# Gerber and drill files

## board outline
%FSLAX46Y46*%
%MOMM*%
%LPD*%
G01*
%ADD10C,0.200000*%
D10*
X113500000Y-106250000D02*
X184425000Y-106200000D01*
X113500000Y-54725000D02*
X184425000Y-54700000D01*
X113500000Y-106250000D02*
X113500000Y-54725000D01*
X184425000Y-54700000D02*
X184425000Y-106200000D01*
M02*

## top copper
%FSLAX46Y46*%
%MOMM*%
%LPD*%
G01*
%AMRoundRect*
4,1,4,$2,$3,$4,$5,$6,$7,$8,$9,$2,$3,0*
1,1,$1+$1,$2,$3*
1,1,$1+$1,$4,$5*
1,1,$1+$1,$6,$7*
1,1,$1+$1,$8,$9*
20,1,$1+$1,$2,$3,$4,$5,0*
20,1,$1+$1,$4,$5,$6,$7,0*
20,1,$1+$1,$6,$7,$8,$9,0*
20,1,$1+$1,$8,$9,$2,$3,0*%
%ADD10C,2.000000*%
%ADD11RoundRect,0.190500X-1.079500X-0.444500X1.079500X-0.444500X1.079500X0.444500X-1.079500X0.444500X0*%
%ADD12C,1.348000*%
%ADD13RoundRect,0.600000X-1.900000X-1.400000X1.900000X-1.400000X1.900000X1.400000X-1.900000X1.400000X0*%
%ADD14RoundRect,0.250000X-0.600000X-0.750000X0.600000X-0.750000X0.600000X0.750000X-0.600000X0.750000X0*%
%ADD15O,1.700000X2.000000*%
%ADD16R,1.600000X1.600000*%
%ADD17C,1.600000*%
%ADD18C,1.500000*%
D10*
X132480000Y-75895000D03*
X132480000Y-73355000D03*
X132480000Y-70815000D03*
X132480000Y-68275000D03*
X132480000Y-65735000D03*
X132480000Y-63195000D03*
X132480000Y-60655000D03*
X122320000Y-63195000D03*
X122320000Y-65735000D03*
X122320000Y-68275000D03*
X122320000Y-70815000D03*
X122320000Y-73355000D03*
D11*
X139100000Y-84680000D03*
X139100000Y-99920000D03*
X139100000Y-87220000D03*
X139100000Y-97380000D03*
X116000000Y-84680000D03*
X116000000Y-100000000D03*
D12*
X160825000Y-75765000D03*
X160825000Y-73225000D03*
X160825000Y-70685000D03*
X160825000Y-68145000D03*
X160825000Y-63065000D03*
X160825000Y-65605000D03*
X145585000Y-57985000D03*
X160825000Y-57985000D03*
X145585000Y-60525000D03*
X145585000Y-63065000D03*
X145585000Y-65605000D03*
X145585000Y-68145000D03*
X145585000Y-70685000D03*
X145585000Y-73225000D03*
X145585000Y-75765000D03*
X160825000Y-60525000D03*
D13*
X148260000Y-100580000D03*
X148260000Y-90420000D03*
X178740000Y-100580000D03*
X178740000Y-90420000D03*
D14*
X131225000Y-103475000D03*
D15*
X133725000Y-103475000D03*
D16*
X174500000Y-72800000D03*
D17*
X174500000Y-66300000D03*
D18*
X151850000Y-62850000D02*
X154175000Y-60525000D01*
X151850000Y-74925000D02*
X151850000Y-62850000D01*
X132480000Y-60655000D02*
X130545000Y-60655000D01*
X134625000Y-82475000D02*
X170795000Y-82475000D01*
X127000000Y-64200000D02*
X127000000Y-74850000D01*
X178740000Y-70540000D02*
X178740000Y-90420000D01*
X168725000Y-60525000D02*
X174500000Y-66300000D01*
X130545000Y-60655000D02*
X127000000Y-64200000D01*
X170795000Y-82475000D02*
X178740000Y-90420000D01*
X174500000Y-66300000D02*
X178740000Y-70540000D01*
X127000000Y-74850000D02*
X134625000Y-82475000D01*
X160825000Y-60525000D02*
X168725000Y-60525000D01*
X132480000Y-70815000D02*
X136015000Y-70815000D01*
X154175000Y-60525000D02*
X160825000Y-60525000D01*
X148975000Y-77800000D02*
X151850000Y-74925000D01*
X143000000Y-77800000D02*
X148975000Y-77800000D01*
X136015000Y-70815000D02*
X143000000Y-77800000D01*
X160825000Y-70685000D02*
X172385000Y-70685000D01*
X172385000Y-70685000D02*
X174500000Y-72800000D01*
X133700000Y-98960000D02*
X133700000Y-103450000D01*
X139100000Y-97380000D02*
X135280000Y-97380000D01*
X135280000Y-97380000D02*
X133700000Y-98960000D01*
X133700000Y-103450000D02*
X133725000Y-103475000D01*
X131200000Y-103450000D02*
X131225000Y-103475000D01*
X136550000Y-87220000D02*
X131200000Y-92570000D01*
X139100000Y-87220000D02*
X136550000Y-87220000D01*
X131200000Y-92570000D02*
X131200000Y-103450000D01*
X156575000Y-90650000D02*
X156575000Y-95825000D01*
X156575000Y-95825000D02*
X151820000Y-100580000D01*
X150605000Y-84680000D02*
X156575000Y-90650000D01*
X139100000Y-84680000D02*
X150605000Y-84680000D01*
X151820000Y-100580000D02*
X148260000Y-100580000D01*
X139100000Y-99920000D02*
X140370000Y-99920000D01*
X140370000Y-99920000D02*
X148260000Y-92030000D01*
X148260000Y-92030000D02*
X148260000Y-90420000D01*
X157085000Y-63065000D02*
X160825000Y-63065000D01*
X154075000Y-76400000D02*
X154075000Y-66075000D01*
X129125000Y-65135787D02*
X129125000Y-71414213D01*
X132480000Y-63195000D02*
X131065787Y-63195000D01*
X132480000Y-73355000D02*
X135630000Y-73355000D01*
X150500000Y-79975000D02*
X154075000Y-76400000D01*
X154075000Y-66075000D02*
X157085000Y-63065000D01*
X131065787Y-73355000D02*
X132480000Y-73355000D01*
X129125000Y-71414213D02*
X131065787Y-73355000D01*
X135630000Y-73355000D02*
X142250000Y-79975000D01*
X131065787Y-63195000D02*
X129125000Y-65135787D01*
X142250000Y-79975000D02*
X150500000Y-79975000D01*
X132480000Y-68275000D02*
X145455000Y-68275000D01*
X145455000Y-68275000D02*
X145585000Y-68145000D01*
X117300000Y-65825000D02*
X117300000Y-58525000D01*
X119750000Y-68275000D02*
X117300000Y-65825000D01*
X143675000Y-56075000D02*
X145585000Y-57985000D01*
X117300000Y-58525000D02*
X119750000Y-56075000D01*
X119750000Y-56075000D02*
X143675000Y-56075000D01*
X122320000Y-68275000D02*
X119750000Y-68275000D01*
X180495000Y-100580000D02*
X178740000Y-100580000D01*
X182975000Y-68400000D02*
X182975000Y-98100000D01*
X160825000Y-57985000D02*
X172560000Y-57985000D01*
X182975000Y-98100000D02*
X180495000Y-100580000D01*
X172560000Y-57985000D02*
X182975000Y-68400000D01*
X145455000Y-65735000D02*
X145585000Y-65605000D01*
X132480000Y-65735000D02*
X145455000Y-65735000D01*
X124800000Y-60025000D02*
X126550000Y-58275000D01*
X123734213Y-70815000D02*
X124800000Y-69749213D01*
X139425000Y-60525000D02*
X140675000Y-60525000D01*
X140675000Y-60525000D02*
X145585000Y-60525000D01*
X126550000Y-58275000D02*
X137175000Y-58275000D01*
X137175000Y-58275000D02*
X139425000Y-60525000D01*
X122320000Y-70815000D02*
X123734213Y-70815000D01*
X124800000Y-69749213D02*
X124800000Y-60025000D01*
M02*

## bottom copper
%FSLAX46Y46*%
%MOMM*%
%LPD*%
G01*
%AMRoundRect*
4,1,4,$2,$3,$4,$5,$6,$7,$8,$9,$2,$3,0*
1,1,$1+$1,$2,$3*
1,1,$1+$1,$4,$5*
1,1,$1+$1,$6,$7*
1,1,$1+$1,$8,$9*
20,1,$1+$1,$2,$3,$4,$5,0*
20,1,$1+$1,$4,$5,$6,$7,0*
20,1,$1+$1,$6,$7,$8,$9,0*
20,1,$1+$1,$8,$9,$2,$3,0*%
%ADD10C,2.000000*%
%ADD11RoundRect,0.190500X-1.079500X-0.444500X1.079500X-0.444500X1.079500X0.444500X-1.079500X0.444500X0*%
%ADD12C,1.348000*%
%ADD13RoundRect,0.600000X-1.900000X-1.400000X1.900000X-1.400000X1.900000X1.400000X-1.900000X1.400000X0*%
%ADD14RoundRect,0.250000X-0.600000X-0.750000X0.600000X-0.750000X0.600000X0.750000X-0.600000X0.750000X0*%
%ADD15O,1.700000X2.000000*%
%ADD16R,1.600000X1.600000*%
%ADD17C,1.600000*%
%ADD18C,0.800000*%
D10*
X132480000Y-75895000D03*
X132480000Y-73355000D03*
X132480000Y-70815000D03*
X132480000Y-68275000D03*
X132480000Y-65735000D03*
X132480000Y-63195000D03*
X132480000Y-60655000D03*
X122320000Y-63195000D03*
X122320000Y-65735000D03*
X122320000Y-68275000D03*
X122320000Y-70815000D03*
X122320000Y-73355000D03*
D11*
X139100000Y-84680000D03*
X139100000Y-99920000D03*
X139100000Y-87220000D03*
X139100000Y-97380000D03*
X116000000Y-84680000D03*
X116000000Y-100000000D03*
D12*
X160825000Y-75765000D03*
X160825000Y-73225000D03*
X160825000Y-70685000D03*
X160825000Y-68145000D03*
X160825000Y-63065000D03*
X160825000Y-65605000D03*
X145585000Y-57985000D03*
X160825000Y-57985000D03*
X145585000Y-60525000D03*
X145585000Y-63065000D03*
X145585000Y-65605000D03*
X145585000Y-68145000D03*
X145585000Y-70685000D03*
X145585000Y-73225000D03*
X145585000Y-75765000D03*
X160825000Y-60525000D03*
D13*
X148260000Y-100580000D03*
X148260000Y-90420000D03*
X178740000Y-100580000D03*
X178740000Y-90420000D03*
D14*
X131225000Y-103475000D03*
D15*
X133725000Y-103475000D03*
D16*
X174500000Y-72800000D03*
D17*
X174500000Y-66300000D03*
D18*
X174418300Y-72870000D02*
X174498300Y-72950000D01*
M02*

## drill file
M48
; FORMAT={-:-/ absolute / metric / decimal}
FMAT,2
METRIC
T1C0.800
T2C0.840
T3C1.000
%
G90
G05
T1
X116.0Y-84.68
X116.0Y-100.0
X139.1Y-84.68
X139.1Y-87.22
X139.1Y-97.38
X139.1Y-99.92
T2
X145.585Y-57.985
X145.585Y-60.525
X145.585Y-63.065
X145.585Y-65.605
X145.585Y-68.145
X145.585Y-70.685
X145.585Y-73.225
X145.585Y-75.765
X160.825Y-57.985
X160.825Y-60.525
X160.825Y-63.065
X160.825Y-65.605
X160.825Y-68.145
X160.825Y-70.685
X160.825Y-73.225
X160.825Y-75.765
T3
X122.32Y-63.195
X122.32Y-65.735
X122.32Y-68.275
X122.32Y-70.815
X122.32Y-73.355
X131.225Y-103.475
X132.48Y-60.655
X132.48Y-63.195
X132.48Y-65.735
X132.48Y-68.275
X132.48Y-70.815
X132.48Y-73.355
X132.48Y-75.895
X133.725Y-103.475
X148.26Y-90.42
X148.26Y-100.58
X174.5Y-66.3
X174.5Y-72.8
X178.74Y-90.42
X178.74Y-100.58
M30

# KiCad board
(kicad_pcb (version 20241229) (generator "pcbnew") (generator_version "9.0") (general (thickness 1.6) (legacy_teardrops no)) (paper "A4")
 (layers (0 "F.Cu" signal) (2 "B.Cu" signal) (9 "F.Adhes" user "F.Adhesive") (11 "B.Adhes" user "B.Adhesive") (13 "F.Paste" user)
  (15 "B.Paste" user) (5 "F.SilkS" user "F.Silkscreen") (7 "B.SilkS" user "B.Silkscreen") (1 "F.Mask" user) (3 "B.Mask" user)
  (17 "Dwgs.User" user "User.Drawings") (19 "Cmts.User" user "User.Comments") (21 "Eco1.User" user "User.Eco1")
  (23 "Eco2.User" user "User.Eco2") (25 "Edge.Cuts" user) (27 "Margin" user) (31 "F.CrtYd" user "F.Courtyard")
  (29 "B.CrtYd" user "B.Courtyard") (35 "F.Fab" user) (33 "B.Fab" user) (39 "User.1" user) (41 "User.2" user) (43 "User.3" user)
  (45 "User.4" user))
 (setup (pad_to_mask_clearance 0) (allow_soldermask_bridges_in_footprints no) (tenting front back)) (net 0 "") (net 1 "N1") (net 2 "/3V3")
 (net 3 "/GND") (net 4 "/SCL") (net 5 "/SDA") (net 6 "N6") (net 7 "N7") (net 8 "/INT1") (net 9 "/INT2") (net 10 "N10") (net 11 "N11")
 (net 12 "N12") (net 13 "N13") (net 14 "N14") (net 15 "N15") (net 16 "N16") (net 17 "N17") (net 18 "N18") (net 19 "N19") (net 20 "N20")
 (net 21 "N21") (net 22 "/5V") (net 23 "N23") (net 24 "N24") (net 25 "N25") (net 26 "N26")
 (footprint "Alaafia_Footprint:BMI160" (layer "F.Cu") (at 127.4 68.275 180)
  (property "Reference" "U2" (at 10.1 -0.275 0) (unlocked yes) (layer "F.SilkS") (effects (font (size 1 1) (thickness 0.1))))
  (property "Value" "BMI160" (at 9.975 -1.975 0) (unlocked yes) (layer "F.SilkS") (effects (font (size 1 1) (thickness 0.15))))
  (pad "1" thru_hole circle (at -5.08 -7.62 180) (size 2 2) (drill 1) (layers "*.Cu" "*.Mask") (remove_unused_layers no) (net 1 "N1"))
  (pad "2" thru_hole circle (at -5.08 -5.08 180) (size 2 2) (drill 1) (layers "*.Cu" "*.Mask") (remove_unused_layers no) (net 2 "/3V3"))
  (pad "3" thru_hole circle (at -5.08 -2.54 180) (size 2 2) (drill 1) (layers "*.Cu" "*.Mask") (remove_unused_layers no) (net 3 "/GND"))
  (pad "4" thru_hole circle (at -5.08 0 180) (size 2 2) (drill 1) (layers "*.Cu" "*.Mask") (remove_unused_layers no) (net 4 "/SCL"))
  (pad "5" thru_hole circle (at -5.08 2.54 180) (size 2 2) (drill 1) (layers "*.Cu" "*.Mask") (remove_unused_layers no) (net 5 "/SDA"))
  (pad "6" thru_hole circle (at -5.08 5.08 180) (size 2 2) (drill 1) (layers "*.Cu" "*.Mask") (remove_unused_layers no) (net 2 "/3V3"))
  (pad "7" thru_hole circle (at -5.08 7.62 180) (size 2 2) (drill 1) (layers "*.Cu" "*.Mask") (remove_unused_layers no) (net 3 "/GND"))
  (pad "8" thru_hole circle (at 5.08 5.08 180) (size 2 2) (drill 1) (layers "*.Cu" "*.Mask") (remove_unused_layers no) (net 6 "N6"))
  (pad "9" thru_hole circle (at 5.08 2.54 180) (size 2 2) (drill 1) (layers "*.Cu" "*.Mask") (remove_unused_layers no) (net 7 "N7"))
  (pad "10" thru_hole circle (at 5.08 0 180) (size 2 2) (drill 1) (layers "*.Cu" "*.Mask") (remove_unused_layers no) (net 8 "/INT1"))
  (pad "11" thru_hole circle (at 5.08 -2.54 180) (size 2 2) (drill 1) (layers "*.Cu" "*.Mask") (remove_unused_layers no) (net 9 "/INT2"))
  (pad "12" thru_hole circle (at 5.08 -5.08 180) (size 2 2) (drill 1) (layers "*.Cu" "*.Mask") (remove_unused_layers no) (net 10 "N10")))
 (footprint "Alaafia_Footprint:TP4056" (layer "F.Cu") (at 128.5 92.3)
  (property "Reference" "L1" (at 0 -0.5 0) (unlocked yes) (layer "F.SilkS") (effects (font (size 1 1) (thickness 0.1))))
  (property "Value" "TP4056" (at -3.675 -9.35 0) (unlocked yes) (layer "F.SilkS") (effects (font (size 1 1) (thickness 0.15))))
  (pad "1" thru_hole roundrect (at 10.6 -7.62) (size 2.54 1.27) (drill 0.8) (layers "*.Cu" "*.Mask") (remove_unused_layers no)
   (roundrect_rratio 0.15) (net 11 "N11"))
  (pad "2" thru_hole roundrect (at 10.6 7.62) (size 2.54 1.27) (drill 0.8) (layers "*.Cu" "*.Mask") (remove_unused_layers no)
   (roundrect_rratio 0.15) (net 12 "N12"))
  (pad "3" thru_hole roundrect (at 10.6 -5.08) (size 2.54 1.27) (drill 0.8) (layers "*.Cu" "*.Mask") (remove_unused_layers no)
   (roundrect_rratio 0.15) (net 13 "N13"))
  (pad "4" thru_hole roundrect (at 10.6 5.08) (size 2.54 1.27) (drill 0.8) (layers "*.Cu" "*.Mask") (remove_unused_layers no)
   (roundrect_rratio 0.15) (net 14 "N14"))
  (pad "5" thru_hole roundrect (at -12.5 -7.62) (size 2.54 1.27) (drill 0.8) (layers "*.Cu" "*.Mask") (remove_unused_layers no)
   (roundrect_rratio 0.15) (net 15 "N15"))
  (pad "6" thru_hole roundrect (at -12.5 7.7) (size 2.54 1.27) (drill 0.8) (layers "*.Cu" "*.Mask") (remove_unused_layers no)
   (roundrect_rratio 0.15) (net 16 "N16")))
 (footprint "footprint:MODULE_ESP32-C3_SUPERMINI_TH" (layer "F.Cu") (at 153.205 67.885)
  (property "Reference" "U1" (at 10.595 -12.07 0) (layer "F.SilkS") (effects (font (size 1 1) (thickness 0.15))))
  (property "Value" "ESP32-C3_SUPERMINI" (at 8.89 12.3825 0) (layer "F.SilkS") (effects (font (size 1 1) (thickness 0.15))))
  (pad "0" thru_hole circle (at 7.62 7.88) (size 1.348 1.348) (drill 0.84) (layers "*.Cu" "*.Mask") (remove_unused_layers no) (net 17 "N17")
   (solder_mask_margin 0.102))
  (pad "1" thru_hole circle (at 7.62 5.34) (size 1.348 1.348) (drill 0.84) (layers "*.Cu" "*.Mask") (remove_unused_layers no) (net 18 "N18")
   (solder_mask_margin 0.102))
  (pad "2" thru_hole circle (at 7.62 2.8) (size 1.348 1.348) (drill 0.84) (layers "*.Cu" "*.Mask") (remove_unused_layers no) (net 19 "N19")
   (solder_mask_margin 0.102))
  (pad "3" thru_hole circle (at 7.62 0.26) (size 1.348 1.348) (drill 0.84) (layers "*.Cu" "*.Mask") (remove_unused_layers no) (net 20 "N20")
   (solder_mask_margin 0.102))
  (pad "3.3" thru_hole circle (at 7.62 -4.82) (size 1.348 1.348) (drill 0.84) (layers "*.Cu" "*.Mask") (remove_unused_layers no)
   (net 2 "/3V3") (solder_mask_margin 0.102))
  (pad "4" thru_hole circle (at 7.62 -2.28) (size 1.348 1.348) (drill 0.84) (layers "*.Cu" "*.Mask") (remove_unused_layers no)
   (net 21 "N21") (solder_mask_margin 0.102))
  (pad "5" thru_hole circle (at -7.62 -9.9) (size 1.348 1.348) (drill 0.84) (layers "*.Cu" "*.Mask") (remove_unused_layers no)
   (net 8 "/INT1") (solder_mask_margin 0.102))
  (pad "5V" thru_hole circle (at 7.62 -9.9) (size 1.348 1.348) (drill 0.84) (layers "*.Cu" "*.Mask") (remove_unused_layers no)
   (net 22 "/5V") (solder_mask_margin 0.102))
  (pad "6" thru_hole circle (at -7.62 -7.36) (size 1.348 1.348) (drill 0.84) (layers "*.Cu" "*.Mask") (remove_unused_layers no)
   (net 9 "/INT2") (solder_mask_margin 0.102))
  (pad "7" thru_hole circle (at -7.62 -4.82) (size 1.348 1.348) (drill 0.84) (layers "*.Cu" "*.Mask") (remove_unused_layers no)
   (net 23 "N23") (solder_mask_margin 0.102))
  (pad "8" thru_hole circle (at -7.62 -2.28) (size 1.348 1.348) (drill 0.84) (layers "*.Cu" "*.Mask") (remove_unused_layers no)
   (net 5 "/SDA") (solder_mask_margin 0.102))
  (pad "9" thru_hole circle (at -7.62 0.26) (size 1.348 1.348) (drill 0.84) (layers "*.Cu" "*.Mask") (remove_unused_layers no)
   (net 4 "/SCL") (solder_mask_margin 0.102))
  (pad "10" thru_hole circle (at -7.62 2.8) (size 1.348 1.348) (drill 0.84) (layers "*.Cu" "*.Mask") (remove_unused_layers no)
   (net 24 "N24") (solder_mask_margin 0.102))
  (pad "20" thru_hole circle (at -7.62 5.34) (size 1.348 1.348) (drill 0.84) (layers "*.Cu" "*.Mask") (remove_unused_layers no)
   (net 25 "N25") (solder_mask_margin 0.102))
  (pad "21" thru_hole circle (at -7.62 7.88) (size 1.348 1.348) (drill 0.84) (layers "*.Cu" "*.Mask") (remove_unused_layers no)
   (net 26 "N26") (solder_mask_margin 0.102))
  (pad "G" thru_hole circle (at 7.62 -7.36) (size 1.348 1.348) (drill 0.84) (layers "*.Cu" "*.Mask") (remove_unused_layers no)
   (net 3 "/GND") (solder_mask_margin 0.102)))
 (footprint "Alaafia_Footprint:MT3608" (layer "F.Cu") (at 163.5 95.5)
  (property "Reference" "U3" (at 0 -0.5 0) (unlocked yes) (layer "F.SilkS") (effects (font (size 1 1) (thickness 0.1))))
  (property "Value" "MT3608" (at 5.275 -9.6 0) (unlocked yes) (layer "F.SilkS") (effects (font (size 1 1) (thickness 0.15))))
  (pad "1" thru_hole roundrect (at -15.24 5.08) (size 5 4) (drill 1) (layers "*.Cu" "*.Mask") (remove_unused_layers no)
   (roundrect_rratio 0.15) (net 11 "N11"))
  (pad "2" thru_hole roundrect (at -15.24 -5.08) (size 5 4) (drill 1) (layers "*.Cu" "*.Mask") (remove_unused_layers no)
   (roundrect_rratio 0.15) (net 12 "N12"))
  (pad "3" thru_hole roundrect (at 15.24 5.08) (size 5 4) (drill 1) (layers "*.Cu" "*.Mask") (remove_unused_layers no)
   (roundrect_rratio 0.15) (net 22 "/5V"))
  (pad "4" thru_hole roundrect (at 15.24 -5.08) (size 5 4) (drill 1) (layers "*.Cu" "*.Mask") (remove_unused_layers no)
   (roundrect_rratio 0.15) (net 3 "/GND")))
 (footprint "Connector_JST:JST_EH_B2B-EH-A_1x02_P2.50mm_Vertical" (layer "F.Cu") (at 131.225 103.475)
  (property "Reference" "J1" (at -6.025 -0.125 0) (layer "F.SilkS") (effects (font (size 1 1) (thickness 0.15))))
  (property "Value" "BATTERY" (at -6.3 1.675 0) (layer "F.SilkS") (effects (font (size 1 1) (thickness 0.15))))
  (pad "1" thru_hole roundrect (at 0 0) (size 1.7 2) (drill 1) (layers "*.Cu" "*.Mask") (remove_unused_layers no)
   (roundrect_rratio 0.147059) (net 13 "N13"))
  (pad "2" thru_hole oval (at 2.5 0) (size 1.7 2) (drill 1) (layers "*.Cu" "*.Mask") (remove_unused_layers no) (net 14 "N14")))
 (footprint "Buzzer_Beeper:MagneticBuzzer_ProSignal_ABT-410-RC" (layer "F.Cu") (at 174.5 72.8 90)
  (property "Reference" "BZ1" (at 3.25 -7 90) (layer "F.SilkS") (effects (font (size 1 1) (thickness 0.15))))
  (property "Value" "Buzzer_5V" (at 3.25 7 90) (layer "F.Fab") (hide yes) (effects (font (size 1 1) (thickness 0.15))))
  (pad "1" thru_hole rect (at 0 0 90) (size 1.6 1.6) (drill 1) (layers "*.Cu" "*.Mask") (remove_unused_layers no) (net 19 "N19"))
  (pad "2" thru_hole circle (at 6.5 0 90) (size 1.6 1.6) (drill 1) (layers "*.Cu" "*.Mask") (remove_unused_layers no) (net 3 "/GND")))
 (gr_line (start 113.5 106.25) (end 184.425 106.2) (stroke (width 0.2) (type solid)) (layer "Edge.Cuts"))
 (gr_line (start 113.5 54.725) (end 184.425 54.7) (stroke (width 0.2) (type solid)) (layer "Edge.Cuts"))
 (gr_line (start 113.5 106.25) (end 113.5 54.725) (stroke (width 0.2) (type solid)) (layer "Edge.Cuts"))
 (gr_line (start 184.425 54.7) (end 184.425 106.2) (stroke (width 0.2) (type solid)) (layer "Edge.Cuts"))
 (segment (start 151.85 62.85) (end 154.175 60.525) (width 1.5) (layer "F.Cu") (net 3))
 (segment (start 151.85 74.925) (end 151.85 62.85) (width 1.5) (layer "F.Cu") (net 3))
 (segment (start 132.48 60.655) (end 130.545 60.655) (width 1.5) (layer "F.Cu") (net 3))
 (segment (start 134.625 82.475) (end 170.795 82.475) (width 1.5) (layer "F.Cu") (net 3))
 (segment (start 127 64.2) (end 127 74.85) (width 1.5) (layer "F.Cu") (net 3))
 (segment (start 178.74 70.54) (end 178.74 90.42) (width 1.5) (layer "F.Cu") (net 3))
 (segment (start 168.725 60.525) (end 174.5 66.3) (width 1.5) (layer "F.Cu") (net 3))
 (segment (start 130.545 60.655) (end 127 64.2) (width 1.5) (layer "F.Cu") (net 3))
 (segment (start 170.795 82.475) (end 178.74 90.42) (width 1.5) (layer "F.Cu") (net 3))
 (segment (start 174.5 66.3) (end 178.74 70.54) (width 1.5) (layer "F.Cu") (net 3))
 (segment (start 127 74.85) (end 134.625 82.475) (width 1.5) (layer "F.Cu") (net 3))
 (segment (start 160.825 60.525) (end 168.725 60.525) (width 1.5) (layer "F.Cu") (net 3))
 (segment (start 132.48 70.815) (end 136.015 70.815) (width 1.5) (layer "F.Cu") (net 3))
 (segment (start 154.175 60.525) (end 160.825 60.525) (width 1.5) (layer "F.Cu") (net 3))
 (segment (start 148.975 77.8) (end 151.85 74.925) (width 1.5) (layer "F.Cu") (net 3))
 (segment (start 143 77.8) (end 148.975 77.8) (width 1.5) (layer "F.Cu") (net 3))
 (segment (start 136.015 70.815) (end 143 77.8) (width 1.5) (layer "F.Cu") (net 3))
 (segment (start 160.825 70.685) (end 172.385 70.685) (width 1.5) (layer "F.Cu") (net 19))
 (segment (start 172.385 70.685) (end 174.5 72.8) (width 1.5) (layer "F.Cu") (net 19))
 (segment (start 174.4183 72.87) (end 174.4983 72.95) (width 0.8) (layer "B.Cu") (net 19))
 (segment (start 133.7 98.96) (end 133.7 103.45) (width 1.5) (layer "F.Cu") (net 14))
 (segment (start 139.1 97.38) (end 135.28 97.38) (width 1.5) (layer "F.Cu") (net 14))
 (segment (start 135.28 97.38) (end 133.7 98.96) (width 1.5) (layer "F.Cu") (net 14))
 (segment (start 133.7 103.45) (end 133.725 103.475) (width 1.5) (layer "F.Cu") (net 14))
 (segment (start 131.2 103.45) (end 131.225 103.475) (width 1.5) (layer "F.Cu") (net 13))
 (segment (start 136.55 87.22) (end 131.2 92.57) (width 1.5) (layer "F.Cu") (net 13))
 (segment (start 139.1 87.22) (end 136.55 87.22) (width 1.5) (layer "F.Cu") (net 13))
 (segment (start 131.2 92.57) (end 131.2 103.45) (width 1.5) (layer "F.Cu") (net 13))
 (segment (start 156.575 90.65) (end 156.575 95.825) (width 1.5) (layer "F.Cu") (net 11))
 (segment (start 156.575 95.825) (end 151.82 100.58) (width 1.5) (layer "F.Cu") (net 11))
 (segment (start 150.605 84.68) (end 156.575 90.65) (width 1.5) (layer "F.Cu") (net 11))
 (segment (start 139.1 84.68) (end 150.605 84.68) (width 1.5) (layer "F.Cu") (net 11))
 (segment (start 151.82 100.58) (end 148.26 100.58) (width 1.5) (layer "F.Cu") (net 11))
 (segment (start 139.1 99.92) (end 140.37 99.92) (width 1.5) (layer "F.Cu") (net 12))
 (segment (start 140.37 99.92) (end 148.26 92.03) (width 1.5) (layer "F.Cu") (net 12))
 (segment (start 148.26 92.03) (end 148.26 90.42) (width 1.5) (layer "F.Cu") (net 12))
 (segment (start 157.085 63.065) (end 160.825 63.065) (width 1.5) (layer "F.Cu") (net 2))
 (segment (start 154.075 76.4) (end 154.075 66.075) (width 1.5) (layer "F.Cu") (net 2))
 (segment (start 129.125 65.135787) (end 129.125 71.414213) (width 1.5) (layer "F.Cu") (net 2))
 (segment (start 132.48 63.195) (end 131.065787 63.195) (width 1.5) (layer "F.Cu") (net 2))
 (segment (start 132.48 73.355) (end 135.63 73.355) (width 1.5) (layer "F.Cu") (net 2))
 (segment (start 150.5 79.975) (end 154.075 76.4) (width 1.5) (layer "F.Cu") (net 2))
 (segment (start 154.075 66.075) (end 157.085 63.065) (width 1.5) (layer "F.Cu") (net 2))
 (segment (start 131.065787 73.355) (end 132.48 73.355) (width 1.5) (layer "F.Cu") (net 2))
 (segment (start 129.125 71.414213) (end 131.065787 73.355) (width 1.5) (layer "F.Cu") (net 2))
 (segment (start 135.63 73.355) (end 142.25 79.975) (width 1.5) (layer "F.Cu") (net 2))
 (segment (start 131.065787 63.195) (end 129.125 65.135787) (width 1.5) (layer "F.Cu") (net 2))
 (segment (start 142.25 79.975) (end 150.5 79.975) (width 1.5) (layer "F.Cu") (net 2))
 (segment (start 132.48 68.275) (end 145.455 68.275) (width 1.5) (layer "F.Cu") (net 4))
 (segment (start 145.455 68.275) (end 145.585 68.145) (width 1.5) (layer "F.Cu") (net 4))
 (segment (start 117.3 65.825) (end 117.3 58.525) (width 1.5) (layer "F.Cu") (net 8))
 (segment (start 119.75 68.275) (end 117.3 65.825) (width 1.5) (layer "F.Cu") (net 8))
 (segment (start 143.675 56.075) (end 145.585 57.985) (width 1.5) (layer "F.Cu") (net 8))
 (segment (start 117.3 58.525) (end 119.75 56.075) (width 1.5) (layer "F.Cu") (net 8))
 (segment (start 119.75 56.075) (end 143.675 56.075) (width 1.5) (layer "F.Cu") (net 8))
 (segment (start 122.32 68.275) (end 119.75 68.275) (width 1.5) (layer "F.Cu") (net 8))
 (segment (start 180.495 100.58) (end 178.74 100.58) (width 1.5) (layer "F.Cu") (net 22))
 (segment (start 182.975 68.4) (end 182.975 98.1) (width 1.5) (layer "F.Cu") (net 22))
 (segment (start 160.825 57.985) (end 172.56 57.985) (width 1.5) (layer "F.Cu") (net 22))
 (segment (start 182.975 98.1) (end 180.495 100.58) (width 1.5) (layer "F.Cu") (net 22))
 (segment (start 172.56 57.985) (end 182.975 68.4) (width 1.5) (layer "F.Cu") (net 22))
 (segment (start 145.455 65.735) (end 145.585 65.605) (width 1.5) (layer "F.Cu") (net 5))
 (segment (start 132.48 65.735) (end 145.455 65.735) (width 1.5) (layer "F.Cu") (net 5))
 (segment (start 124.8 60.025) (end 126.55 58.275) (width 1.5) (layer "F.Cu") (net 9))
 (segment (start 123.734213 70.815) (end 124.8 69.749213) (width 1.5) (layer "F.Cu") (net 9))
 (segment (start 139.425 60.525) (end 140.675 60.525) (width 1.5) (layer "F.Cu") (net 9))
 (segment (start 140.675 60.525) (end 145.585 60.525) (width 1.5) (layer "F.Cu") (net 9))
 (segment (start 126.55 58.275) (end 137.175 58.275) (width 1.5) (layer "F.Cu") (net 9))
 (segment (start 137.175 58.275) (end 139.425 60.525) (width 1.5) (layer "F.Cu") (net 9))
 (segment (start 122.32 70.815) (end 123.734213 70.815) (width 1.5) (layer "F.Cu") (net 9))
 (segment (start 124.8 69.749213) (end 124.8 60.025) (width 1.5) (layer "F.Cu") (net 9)))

